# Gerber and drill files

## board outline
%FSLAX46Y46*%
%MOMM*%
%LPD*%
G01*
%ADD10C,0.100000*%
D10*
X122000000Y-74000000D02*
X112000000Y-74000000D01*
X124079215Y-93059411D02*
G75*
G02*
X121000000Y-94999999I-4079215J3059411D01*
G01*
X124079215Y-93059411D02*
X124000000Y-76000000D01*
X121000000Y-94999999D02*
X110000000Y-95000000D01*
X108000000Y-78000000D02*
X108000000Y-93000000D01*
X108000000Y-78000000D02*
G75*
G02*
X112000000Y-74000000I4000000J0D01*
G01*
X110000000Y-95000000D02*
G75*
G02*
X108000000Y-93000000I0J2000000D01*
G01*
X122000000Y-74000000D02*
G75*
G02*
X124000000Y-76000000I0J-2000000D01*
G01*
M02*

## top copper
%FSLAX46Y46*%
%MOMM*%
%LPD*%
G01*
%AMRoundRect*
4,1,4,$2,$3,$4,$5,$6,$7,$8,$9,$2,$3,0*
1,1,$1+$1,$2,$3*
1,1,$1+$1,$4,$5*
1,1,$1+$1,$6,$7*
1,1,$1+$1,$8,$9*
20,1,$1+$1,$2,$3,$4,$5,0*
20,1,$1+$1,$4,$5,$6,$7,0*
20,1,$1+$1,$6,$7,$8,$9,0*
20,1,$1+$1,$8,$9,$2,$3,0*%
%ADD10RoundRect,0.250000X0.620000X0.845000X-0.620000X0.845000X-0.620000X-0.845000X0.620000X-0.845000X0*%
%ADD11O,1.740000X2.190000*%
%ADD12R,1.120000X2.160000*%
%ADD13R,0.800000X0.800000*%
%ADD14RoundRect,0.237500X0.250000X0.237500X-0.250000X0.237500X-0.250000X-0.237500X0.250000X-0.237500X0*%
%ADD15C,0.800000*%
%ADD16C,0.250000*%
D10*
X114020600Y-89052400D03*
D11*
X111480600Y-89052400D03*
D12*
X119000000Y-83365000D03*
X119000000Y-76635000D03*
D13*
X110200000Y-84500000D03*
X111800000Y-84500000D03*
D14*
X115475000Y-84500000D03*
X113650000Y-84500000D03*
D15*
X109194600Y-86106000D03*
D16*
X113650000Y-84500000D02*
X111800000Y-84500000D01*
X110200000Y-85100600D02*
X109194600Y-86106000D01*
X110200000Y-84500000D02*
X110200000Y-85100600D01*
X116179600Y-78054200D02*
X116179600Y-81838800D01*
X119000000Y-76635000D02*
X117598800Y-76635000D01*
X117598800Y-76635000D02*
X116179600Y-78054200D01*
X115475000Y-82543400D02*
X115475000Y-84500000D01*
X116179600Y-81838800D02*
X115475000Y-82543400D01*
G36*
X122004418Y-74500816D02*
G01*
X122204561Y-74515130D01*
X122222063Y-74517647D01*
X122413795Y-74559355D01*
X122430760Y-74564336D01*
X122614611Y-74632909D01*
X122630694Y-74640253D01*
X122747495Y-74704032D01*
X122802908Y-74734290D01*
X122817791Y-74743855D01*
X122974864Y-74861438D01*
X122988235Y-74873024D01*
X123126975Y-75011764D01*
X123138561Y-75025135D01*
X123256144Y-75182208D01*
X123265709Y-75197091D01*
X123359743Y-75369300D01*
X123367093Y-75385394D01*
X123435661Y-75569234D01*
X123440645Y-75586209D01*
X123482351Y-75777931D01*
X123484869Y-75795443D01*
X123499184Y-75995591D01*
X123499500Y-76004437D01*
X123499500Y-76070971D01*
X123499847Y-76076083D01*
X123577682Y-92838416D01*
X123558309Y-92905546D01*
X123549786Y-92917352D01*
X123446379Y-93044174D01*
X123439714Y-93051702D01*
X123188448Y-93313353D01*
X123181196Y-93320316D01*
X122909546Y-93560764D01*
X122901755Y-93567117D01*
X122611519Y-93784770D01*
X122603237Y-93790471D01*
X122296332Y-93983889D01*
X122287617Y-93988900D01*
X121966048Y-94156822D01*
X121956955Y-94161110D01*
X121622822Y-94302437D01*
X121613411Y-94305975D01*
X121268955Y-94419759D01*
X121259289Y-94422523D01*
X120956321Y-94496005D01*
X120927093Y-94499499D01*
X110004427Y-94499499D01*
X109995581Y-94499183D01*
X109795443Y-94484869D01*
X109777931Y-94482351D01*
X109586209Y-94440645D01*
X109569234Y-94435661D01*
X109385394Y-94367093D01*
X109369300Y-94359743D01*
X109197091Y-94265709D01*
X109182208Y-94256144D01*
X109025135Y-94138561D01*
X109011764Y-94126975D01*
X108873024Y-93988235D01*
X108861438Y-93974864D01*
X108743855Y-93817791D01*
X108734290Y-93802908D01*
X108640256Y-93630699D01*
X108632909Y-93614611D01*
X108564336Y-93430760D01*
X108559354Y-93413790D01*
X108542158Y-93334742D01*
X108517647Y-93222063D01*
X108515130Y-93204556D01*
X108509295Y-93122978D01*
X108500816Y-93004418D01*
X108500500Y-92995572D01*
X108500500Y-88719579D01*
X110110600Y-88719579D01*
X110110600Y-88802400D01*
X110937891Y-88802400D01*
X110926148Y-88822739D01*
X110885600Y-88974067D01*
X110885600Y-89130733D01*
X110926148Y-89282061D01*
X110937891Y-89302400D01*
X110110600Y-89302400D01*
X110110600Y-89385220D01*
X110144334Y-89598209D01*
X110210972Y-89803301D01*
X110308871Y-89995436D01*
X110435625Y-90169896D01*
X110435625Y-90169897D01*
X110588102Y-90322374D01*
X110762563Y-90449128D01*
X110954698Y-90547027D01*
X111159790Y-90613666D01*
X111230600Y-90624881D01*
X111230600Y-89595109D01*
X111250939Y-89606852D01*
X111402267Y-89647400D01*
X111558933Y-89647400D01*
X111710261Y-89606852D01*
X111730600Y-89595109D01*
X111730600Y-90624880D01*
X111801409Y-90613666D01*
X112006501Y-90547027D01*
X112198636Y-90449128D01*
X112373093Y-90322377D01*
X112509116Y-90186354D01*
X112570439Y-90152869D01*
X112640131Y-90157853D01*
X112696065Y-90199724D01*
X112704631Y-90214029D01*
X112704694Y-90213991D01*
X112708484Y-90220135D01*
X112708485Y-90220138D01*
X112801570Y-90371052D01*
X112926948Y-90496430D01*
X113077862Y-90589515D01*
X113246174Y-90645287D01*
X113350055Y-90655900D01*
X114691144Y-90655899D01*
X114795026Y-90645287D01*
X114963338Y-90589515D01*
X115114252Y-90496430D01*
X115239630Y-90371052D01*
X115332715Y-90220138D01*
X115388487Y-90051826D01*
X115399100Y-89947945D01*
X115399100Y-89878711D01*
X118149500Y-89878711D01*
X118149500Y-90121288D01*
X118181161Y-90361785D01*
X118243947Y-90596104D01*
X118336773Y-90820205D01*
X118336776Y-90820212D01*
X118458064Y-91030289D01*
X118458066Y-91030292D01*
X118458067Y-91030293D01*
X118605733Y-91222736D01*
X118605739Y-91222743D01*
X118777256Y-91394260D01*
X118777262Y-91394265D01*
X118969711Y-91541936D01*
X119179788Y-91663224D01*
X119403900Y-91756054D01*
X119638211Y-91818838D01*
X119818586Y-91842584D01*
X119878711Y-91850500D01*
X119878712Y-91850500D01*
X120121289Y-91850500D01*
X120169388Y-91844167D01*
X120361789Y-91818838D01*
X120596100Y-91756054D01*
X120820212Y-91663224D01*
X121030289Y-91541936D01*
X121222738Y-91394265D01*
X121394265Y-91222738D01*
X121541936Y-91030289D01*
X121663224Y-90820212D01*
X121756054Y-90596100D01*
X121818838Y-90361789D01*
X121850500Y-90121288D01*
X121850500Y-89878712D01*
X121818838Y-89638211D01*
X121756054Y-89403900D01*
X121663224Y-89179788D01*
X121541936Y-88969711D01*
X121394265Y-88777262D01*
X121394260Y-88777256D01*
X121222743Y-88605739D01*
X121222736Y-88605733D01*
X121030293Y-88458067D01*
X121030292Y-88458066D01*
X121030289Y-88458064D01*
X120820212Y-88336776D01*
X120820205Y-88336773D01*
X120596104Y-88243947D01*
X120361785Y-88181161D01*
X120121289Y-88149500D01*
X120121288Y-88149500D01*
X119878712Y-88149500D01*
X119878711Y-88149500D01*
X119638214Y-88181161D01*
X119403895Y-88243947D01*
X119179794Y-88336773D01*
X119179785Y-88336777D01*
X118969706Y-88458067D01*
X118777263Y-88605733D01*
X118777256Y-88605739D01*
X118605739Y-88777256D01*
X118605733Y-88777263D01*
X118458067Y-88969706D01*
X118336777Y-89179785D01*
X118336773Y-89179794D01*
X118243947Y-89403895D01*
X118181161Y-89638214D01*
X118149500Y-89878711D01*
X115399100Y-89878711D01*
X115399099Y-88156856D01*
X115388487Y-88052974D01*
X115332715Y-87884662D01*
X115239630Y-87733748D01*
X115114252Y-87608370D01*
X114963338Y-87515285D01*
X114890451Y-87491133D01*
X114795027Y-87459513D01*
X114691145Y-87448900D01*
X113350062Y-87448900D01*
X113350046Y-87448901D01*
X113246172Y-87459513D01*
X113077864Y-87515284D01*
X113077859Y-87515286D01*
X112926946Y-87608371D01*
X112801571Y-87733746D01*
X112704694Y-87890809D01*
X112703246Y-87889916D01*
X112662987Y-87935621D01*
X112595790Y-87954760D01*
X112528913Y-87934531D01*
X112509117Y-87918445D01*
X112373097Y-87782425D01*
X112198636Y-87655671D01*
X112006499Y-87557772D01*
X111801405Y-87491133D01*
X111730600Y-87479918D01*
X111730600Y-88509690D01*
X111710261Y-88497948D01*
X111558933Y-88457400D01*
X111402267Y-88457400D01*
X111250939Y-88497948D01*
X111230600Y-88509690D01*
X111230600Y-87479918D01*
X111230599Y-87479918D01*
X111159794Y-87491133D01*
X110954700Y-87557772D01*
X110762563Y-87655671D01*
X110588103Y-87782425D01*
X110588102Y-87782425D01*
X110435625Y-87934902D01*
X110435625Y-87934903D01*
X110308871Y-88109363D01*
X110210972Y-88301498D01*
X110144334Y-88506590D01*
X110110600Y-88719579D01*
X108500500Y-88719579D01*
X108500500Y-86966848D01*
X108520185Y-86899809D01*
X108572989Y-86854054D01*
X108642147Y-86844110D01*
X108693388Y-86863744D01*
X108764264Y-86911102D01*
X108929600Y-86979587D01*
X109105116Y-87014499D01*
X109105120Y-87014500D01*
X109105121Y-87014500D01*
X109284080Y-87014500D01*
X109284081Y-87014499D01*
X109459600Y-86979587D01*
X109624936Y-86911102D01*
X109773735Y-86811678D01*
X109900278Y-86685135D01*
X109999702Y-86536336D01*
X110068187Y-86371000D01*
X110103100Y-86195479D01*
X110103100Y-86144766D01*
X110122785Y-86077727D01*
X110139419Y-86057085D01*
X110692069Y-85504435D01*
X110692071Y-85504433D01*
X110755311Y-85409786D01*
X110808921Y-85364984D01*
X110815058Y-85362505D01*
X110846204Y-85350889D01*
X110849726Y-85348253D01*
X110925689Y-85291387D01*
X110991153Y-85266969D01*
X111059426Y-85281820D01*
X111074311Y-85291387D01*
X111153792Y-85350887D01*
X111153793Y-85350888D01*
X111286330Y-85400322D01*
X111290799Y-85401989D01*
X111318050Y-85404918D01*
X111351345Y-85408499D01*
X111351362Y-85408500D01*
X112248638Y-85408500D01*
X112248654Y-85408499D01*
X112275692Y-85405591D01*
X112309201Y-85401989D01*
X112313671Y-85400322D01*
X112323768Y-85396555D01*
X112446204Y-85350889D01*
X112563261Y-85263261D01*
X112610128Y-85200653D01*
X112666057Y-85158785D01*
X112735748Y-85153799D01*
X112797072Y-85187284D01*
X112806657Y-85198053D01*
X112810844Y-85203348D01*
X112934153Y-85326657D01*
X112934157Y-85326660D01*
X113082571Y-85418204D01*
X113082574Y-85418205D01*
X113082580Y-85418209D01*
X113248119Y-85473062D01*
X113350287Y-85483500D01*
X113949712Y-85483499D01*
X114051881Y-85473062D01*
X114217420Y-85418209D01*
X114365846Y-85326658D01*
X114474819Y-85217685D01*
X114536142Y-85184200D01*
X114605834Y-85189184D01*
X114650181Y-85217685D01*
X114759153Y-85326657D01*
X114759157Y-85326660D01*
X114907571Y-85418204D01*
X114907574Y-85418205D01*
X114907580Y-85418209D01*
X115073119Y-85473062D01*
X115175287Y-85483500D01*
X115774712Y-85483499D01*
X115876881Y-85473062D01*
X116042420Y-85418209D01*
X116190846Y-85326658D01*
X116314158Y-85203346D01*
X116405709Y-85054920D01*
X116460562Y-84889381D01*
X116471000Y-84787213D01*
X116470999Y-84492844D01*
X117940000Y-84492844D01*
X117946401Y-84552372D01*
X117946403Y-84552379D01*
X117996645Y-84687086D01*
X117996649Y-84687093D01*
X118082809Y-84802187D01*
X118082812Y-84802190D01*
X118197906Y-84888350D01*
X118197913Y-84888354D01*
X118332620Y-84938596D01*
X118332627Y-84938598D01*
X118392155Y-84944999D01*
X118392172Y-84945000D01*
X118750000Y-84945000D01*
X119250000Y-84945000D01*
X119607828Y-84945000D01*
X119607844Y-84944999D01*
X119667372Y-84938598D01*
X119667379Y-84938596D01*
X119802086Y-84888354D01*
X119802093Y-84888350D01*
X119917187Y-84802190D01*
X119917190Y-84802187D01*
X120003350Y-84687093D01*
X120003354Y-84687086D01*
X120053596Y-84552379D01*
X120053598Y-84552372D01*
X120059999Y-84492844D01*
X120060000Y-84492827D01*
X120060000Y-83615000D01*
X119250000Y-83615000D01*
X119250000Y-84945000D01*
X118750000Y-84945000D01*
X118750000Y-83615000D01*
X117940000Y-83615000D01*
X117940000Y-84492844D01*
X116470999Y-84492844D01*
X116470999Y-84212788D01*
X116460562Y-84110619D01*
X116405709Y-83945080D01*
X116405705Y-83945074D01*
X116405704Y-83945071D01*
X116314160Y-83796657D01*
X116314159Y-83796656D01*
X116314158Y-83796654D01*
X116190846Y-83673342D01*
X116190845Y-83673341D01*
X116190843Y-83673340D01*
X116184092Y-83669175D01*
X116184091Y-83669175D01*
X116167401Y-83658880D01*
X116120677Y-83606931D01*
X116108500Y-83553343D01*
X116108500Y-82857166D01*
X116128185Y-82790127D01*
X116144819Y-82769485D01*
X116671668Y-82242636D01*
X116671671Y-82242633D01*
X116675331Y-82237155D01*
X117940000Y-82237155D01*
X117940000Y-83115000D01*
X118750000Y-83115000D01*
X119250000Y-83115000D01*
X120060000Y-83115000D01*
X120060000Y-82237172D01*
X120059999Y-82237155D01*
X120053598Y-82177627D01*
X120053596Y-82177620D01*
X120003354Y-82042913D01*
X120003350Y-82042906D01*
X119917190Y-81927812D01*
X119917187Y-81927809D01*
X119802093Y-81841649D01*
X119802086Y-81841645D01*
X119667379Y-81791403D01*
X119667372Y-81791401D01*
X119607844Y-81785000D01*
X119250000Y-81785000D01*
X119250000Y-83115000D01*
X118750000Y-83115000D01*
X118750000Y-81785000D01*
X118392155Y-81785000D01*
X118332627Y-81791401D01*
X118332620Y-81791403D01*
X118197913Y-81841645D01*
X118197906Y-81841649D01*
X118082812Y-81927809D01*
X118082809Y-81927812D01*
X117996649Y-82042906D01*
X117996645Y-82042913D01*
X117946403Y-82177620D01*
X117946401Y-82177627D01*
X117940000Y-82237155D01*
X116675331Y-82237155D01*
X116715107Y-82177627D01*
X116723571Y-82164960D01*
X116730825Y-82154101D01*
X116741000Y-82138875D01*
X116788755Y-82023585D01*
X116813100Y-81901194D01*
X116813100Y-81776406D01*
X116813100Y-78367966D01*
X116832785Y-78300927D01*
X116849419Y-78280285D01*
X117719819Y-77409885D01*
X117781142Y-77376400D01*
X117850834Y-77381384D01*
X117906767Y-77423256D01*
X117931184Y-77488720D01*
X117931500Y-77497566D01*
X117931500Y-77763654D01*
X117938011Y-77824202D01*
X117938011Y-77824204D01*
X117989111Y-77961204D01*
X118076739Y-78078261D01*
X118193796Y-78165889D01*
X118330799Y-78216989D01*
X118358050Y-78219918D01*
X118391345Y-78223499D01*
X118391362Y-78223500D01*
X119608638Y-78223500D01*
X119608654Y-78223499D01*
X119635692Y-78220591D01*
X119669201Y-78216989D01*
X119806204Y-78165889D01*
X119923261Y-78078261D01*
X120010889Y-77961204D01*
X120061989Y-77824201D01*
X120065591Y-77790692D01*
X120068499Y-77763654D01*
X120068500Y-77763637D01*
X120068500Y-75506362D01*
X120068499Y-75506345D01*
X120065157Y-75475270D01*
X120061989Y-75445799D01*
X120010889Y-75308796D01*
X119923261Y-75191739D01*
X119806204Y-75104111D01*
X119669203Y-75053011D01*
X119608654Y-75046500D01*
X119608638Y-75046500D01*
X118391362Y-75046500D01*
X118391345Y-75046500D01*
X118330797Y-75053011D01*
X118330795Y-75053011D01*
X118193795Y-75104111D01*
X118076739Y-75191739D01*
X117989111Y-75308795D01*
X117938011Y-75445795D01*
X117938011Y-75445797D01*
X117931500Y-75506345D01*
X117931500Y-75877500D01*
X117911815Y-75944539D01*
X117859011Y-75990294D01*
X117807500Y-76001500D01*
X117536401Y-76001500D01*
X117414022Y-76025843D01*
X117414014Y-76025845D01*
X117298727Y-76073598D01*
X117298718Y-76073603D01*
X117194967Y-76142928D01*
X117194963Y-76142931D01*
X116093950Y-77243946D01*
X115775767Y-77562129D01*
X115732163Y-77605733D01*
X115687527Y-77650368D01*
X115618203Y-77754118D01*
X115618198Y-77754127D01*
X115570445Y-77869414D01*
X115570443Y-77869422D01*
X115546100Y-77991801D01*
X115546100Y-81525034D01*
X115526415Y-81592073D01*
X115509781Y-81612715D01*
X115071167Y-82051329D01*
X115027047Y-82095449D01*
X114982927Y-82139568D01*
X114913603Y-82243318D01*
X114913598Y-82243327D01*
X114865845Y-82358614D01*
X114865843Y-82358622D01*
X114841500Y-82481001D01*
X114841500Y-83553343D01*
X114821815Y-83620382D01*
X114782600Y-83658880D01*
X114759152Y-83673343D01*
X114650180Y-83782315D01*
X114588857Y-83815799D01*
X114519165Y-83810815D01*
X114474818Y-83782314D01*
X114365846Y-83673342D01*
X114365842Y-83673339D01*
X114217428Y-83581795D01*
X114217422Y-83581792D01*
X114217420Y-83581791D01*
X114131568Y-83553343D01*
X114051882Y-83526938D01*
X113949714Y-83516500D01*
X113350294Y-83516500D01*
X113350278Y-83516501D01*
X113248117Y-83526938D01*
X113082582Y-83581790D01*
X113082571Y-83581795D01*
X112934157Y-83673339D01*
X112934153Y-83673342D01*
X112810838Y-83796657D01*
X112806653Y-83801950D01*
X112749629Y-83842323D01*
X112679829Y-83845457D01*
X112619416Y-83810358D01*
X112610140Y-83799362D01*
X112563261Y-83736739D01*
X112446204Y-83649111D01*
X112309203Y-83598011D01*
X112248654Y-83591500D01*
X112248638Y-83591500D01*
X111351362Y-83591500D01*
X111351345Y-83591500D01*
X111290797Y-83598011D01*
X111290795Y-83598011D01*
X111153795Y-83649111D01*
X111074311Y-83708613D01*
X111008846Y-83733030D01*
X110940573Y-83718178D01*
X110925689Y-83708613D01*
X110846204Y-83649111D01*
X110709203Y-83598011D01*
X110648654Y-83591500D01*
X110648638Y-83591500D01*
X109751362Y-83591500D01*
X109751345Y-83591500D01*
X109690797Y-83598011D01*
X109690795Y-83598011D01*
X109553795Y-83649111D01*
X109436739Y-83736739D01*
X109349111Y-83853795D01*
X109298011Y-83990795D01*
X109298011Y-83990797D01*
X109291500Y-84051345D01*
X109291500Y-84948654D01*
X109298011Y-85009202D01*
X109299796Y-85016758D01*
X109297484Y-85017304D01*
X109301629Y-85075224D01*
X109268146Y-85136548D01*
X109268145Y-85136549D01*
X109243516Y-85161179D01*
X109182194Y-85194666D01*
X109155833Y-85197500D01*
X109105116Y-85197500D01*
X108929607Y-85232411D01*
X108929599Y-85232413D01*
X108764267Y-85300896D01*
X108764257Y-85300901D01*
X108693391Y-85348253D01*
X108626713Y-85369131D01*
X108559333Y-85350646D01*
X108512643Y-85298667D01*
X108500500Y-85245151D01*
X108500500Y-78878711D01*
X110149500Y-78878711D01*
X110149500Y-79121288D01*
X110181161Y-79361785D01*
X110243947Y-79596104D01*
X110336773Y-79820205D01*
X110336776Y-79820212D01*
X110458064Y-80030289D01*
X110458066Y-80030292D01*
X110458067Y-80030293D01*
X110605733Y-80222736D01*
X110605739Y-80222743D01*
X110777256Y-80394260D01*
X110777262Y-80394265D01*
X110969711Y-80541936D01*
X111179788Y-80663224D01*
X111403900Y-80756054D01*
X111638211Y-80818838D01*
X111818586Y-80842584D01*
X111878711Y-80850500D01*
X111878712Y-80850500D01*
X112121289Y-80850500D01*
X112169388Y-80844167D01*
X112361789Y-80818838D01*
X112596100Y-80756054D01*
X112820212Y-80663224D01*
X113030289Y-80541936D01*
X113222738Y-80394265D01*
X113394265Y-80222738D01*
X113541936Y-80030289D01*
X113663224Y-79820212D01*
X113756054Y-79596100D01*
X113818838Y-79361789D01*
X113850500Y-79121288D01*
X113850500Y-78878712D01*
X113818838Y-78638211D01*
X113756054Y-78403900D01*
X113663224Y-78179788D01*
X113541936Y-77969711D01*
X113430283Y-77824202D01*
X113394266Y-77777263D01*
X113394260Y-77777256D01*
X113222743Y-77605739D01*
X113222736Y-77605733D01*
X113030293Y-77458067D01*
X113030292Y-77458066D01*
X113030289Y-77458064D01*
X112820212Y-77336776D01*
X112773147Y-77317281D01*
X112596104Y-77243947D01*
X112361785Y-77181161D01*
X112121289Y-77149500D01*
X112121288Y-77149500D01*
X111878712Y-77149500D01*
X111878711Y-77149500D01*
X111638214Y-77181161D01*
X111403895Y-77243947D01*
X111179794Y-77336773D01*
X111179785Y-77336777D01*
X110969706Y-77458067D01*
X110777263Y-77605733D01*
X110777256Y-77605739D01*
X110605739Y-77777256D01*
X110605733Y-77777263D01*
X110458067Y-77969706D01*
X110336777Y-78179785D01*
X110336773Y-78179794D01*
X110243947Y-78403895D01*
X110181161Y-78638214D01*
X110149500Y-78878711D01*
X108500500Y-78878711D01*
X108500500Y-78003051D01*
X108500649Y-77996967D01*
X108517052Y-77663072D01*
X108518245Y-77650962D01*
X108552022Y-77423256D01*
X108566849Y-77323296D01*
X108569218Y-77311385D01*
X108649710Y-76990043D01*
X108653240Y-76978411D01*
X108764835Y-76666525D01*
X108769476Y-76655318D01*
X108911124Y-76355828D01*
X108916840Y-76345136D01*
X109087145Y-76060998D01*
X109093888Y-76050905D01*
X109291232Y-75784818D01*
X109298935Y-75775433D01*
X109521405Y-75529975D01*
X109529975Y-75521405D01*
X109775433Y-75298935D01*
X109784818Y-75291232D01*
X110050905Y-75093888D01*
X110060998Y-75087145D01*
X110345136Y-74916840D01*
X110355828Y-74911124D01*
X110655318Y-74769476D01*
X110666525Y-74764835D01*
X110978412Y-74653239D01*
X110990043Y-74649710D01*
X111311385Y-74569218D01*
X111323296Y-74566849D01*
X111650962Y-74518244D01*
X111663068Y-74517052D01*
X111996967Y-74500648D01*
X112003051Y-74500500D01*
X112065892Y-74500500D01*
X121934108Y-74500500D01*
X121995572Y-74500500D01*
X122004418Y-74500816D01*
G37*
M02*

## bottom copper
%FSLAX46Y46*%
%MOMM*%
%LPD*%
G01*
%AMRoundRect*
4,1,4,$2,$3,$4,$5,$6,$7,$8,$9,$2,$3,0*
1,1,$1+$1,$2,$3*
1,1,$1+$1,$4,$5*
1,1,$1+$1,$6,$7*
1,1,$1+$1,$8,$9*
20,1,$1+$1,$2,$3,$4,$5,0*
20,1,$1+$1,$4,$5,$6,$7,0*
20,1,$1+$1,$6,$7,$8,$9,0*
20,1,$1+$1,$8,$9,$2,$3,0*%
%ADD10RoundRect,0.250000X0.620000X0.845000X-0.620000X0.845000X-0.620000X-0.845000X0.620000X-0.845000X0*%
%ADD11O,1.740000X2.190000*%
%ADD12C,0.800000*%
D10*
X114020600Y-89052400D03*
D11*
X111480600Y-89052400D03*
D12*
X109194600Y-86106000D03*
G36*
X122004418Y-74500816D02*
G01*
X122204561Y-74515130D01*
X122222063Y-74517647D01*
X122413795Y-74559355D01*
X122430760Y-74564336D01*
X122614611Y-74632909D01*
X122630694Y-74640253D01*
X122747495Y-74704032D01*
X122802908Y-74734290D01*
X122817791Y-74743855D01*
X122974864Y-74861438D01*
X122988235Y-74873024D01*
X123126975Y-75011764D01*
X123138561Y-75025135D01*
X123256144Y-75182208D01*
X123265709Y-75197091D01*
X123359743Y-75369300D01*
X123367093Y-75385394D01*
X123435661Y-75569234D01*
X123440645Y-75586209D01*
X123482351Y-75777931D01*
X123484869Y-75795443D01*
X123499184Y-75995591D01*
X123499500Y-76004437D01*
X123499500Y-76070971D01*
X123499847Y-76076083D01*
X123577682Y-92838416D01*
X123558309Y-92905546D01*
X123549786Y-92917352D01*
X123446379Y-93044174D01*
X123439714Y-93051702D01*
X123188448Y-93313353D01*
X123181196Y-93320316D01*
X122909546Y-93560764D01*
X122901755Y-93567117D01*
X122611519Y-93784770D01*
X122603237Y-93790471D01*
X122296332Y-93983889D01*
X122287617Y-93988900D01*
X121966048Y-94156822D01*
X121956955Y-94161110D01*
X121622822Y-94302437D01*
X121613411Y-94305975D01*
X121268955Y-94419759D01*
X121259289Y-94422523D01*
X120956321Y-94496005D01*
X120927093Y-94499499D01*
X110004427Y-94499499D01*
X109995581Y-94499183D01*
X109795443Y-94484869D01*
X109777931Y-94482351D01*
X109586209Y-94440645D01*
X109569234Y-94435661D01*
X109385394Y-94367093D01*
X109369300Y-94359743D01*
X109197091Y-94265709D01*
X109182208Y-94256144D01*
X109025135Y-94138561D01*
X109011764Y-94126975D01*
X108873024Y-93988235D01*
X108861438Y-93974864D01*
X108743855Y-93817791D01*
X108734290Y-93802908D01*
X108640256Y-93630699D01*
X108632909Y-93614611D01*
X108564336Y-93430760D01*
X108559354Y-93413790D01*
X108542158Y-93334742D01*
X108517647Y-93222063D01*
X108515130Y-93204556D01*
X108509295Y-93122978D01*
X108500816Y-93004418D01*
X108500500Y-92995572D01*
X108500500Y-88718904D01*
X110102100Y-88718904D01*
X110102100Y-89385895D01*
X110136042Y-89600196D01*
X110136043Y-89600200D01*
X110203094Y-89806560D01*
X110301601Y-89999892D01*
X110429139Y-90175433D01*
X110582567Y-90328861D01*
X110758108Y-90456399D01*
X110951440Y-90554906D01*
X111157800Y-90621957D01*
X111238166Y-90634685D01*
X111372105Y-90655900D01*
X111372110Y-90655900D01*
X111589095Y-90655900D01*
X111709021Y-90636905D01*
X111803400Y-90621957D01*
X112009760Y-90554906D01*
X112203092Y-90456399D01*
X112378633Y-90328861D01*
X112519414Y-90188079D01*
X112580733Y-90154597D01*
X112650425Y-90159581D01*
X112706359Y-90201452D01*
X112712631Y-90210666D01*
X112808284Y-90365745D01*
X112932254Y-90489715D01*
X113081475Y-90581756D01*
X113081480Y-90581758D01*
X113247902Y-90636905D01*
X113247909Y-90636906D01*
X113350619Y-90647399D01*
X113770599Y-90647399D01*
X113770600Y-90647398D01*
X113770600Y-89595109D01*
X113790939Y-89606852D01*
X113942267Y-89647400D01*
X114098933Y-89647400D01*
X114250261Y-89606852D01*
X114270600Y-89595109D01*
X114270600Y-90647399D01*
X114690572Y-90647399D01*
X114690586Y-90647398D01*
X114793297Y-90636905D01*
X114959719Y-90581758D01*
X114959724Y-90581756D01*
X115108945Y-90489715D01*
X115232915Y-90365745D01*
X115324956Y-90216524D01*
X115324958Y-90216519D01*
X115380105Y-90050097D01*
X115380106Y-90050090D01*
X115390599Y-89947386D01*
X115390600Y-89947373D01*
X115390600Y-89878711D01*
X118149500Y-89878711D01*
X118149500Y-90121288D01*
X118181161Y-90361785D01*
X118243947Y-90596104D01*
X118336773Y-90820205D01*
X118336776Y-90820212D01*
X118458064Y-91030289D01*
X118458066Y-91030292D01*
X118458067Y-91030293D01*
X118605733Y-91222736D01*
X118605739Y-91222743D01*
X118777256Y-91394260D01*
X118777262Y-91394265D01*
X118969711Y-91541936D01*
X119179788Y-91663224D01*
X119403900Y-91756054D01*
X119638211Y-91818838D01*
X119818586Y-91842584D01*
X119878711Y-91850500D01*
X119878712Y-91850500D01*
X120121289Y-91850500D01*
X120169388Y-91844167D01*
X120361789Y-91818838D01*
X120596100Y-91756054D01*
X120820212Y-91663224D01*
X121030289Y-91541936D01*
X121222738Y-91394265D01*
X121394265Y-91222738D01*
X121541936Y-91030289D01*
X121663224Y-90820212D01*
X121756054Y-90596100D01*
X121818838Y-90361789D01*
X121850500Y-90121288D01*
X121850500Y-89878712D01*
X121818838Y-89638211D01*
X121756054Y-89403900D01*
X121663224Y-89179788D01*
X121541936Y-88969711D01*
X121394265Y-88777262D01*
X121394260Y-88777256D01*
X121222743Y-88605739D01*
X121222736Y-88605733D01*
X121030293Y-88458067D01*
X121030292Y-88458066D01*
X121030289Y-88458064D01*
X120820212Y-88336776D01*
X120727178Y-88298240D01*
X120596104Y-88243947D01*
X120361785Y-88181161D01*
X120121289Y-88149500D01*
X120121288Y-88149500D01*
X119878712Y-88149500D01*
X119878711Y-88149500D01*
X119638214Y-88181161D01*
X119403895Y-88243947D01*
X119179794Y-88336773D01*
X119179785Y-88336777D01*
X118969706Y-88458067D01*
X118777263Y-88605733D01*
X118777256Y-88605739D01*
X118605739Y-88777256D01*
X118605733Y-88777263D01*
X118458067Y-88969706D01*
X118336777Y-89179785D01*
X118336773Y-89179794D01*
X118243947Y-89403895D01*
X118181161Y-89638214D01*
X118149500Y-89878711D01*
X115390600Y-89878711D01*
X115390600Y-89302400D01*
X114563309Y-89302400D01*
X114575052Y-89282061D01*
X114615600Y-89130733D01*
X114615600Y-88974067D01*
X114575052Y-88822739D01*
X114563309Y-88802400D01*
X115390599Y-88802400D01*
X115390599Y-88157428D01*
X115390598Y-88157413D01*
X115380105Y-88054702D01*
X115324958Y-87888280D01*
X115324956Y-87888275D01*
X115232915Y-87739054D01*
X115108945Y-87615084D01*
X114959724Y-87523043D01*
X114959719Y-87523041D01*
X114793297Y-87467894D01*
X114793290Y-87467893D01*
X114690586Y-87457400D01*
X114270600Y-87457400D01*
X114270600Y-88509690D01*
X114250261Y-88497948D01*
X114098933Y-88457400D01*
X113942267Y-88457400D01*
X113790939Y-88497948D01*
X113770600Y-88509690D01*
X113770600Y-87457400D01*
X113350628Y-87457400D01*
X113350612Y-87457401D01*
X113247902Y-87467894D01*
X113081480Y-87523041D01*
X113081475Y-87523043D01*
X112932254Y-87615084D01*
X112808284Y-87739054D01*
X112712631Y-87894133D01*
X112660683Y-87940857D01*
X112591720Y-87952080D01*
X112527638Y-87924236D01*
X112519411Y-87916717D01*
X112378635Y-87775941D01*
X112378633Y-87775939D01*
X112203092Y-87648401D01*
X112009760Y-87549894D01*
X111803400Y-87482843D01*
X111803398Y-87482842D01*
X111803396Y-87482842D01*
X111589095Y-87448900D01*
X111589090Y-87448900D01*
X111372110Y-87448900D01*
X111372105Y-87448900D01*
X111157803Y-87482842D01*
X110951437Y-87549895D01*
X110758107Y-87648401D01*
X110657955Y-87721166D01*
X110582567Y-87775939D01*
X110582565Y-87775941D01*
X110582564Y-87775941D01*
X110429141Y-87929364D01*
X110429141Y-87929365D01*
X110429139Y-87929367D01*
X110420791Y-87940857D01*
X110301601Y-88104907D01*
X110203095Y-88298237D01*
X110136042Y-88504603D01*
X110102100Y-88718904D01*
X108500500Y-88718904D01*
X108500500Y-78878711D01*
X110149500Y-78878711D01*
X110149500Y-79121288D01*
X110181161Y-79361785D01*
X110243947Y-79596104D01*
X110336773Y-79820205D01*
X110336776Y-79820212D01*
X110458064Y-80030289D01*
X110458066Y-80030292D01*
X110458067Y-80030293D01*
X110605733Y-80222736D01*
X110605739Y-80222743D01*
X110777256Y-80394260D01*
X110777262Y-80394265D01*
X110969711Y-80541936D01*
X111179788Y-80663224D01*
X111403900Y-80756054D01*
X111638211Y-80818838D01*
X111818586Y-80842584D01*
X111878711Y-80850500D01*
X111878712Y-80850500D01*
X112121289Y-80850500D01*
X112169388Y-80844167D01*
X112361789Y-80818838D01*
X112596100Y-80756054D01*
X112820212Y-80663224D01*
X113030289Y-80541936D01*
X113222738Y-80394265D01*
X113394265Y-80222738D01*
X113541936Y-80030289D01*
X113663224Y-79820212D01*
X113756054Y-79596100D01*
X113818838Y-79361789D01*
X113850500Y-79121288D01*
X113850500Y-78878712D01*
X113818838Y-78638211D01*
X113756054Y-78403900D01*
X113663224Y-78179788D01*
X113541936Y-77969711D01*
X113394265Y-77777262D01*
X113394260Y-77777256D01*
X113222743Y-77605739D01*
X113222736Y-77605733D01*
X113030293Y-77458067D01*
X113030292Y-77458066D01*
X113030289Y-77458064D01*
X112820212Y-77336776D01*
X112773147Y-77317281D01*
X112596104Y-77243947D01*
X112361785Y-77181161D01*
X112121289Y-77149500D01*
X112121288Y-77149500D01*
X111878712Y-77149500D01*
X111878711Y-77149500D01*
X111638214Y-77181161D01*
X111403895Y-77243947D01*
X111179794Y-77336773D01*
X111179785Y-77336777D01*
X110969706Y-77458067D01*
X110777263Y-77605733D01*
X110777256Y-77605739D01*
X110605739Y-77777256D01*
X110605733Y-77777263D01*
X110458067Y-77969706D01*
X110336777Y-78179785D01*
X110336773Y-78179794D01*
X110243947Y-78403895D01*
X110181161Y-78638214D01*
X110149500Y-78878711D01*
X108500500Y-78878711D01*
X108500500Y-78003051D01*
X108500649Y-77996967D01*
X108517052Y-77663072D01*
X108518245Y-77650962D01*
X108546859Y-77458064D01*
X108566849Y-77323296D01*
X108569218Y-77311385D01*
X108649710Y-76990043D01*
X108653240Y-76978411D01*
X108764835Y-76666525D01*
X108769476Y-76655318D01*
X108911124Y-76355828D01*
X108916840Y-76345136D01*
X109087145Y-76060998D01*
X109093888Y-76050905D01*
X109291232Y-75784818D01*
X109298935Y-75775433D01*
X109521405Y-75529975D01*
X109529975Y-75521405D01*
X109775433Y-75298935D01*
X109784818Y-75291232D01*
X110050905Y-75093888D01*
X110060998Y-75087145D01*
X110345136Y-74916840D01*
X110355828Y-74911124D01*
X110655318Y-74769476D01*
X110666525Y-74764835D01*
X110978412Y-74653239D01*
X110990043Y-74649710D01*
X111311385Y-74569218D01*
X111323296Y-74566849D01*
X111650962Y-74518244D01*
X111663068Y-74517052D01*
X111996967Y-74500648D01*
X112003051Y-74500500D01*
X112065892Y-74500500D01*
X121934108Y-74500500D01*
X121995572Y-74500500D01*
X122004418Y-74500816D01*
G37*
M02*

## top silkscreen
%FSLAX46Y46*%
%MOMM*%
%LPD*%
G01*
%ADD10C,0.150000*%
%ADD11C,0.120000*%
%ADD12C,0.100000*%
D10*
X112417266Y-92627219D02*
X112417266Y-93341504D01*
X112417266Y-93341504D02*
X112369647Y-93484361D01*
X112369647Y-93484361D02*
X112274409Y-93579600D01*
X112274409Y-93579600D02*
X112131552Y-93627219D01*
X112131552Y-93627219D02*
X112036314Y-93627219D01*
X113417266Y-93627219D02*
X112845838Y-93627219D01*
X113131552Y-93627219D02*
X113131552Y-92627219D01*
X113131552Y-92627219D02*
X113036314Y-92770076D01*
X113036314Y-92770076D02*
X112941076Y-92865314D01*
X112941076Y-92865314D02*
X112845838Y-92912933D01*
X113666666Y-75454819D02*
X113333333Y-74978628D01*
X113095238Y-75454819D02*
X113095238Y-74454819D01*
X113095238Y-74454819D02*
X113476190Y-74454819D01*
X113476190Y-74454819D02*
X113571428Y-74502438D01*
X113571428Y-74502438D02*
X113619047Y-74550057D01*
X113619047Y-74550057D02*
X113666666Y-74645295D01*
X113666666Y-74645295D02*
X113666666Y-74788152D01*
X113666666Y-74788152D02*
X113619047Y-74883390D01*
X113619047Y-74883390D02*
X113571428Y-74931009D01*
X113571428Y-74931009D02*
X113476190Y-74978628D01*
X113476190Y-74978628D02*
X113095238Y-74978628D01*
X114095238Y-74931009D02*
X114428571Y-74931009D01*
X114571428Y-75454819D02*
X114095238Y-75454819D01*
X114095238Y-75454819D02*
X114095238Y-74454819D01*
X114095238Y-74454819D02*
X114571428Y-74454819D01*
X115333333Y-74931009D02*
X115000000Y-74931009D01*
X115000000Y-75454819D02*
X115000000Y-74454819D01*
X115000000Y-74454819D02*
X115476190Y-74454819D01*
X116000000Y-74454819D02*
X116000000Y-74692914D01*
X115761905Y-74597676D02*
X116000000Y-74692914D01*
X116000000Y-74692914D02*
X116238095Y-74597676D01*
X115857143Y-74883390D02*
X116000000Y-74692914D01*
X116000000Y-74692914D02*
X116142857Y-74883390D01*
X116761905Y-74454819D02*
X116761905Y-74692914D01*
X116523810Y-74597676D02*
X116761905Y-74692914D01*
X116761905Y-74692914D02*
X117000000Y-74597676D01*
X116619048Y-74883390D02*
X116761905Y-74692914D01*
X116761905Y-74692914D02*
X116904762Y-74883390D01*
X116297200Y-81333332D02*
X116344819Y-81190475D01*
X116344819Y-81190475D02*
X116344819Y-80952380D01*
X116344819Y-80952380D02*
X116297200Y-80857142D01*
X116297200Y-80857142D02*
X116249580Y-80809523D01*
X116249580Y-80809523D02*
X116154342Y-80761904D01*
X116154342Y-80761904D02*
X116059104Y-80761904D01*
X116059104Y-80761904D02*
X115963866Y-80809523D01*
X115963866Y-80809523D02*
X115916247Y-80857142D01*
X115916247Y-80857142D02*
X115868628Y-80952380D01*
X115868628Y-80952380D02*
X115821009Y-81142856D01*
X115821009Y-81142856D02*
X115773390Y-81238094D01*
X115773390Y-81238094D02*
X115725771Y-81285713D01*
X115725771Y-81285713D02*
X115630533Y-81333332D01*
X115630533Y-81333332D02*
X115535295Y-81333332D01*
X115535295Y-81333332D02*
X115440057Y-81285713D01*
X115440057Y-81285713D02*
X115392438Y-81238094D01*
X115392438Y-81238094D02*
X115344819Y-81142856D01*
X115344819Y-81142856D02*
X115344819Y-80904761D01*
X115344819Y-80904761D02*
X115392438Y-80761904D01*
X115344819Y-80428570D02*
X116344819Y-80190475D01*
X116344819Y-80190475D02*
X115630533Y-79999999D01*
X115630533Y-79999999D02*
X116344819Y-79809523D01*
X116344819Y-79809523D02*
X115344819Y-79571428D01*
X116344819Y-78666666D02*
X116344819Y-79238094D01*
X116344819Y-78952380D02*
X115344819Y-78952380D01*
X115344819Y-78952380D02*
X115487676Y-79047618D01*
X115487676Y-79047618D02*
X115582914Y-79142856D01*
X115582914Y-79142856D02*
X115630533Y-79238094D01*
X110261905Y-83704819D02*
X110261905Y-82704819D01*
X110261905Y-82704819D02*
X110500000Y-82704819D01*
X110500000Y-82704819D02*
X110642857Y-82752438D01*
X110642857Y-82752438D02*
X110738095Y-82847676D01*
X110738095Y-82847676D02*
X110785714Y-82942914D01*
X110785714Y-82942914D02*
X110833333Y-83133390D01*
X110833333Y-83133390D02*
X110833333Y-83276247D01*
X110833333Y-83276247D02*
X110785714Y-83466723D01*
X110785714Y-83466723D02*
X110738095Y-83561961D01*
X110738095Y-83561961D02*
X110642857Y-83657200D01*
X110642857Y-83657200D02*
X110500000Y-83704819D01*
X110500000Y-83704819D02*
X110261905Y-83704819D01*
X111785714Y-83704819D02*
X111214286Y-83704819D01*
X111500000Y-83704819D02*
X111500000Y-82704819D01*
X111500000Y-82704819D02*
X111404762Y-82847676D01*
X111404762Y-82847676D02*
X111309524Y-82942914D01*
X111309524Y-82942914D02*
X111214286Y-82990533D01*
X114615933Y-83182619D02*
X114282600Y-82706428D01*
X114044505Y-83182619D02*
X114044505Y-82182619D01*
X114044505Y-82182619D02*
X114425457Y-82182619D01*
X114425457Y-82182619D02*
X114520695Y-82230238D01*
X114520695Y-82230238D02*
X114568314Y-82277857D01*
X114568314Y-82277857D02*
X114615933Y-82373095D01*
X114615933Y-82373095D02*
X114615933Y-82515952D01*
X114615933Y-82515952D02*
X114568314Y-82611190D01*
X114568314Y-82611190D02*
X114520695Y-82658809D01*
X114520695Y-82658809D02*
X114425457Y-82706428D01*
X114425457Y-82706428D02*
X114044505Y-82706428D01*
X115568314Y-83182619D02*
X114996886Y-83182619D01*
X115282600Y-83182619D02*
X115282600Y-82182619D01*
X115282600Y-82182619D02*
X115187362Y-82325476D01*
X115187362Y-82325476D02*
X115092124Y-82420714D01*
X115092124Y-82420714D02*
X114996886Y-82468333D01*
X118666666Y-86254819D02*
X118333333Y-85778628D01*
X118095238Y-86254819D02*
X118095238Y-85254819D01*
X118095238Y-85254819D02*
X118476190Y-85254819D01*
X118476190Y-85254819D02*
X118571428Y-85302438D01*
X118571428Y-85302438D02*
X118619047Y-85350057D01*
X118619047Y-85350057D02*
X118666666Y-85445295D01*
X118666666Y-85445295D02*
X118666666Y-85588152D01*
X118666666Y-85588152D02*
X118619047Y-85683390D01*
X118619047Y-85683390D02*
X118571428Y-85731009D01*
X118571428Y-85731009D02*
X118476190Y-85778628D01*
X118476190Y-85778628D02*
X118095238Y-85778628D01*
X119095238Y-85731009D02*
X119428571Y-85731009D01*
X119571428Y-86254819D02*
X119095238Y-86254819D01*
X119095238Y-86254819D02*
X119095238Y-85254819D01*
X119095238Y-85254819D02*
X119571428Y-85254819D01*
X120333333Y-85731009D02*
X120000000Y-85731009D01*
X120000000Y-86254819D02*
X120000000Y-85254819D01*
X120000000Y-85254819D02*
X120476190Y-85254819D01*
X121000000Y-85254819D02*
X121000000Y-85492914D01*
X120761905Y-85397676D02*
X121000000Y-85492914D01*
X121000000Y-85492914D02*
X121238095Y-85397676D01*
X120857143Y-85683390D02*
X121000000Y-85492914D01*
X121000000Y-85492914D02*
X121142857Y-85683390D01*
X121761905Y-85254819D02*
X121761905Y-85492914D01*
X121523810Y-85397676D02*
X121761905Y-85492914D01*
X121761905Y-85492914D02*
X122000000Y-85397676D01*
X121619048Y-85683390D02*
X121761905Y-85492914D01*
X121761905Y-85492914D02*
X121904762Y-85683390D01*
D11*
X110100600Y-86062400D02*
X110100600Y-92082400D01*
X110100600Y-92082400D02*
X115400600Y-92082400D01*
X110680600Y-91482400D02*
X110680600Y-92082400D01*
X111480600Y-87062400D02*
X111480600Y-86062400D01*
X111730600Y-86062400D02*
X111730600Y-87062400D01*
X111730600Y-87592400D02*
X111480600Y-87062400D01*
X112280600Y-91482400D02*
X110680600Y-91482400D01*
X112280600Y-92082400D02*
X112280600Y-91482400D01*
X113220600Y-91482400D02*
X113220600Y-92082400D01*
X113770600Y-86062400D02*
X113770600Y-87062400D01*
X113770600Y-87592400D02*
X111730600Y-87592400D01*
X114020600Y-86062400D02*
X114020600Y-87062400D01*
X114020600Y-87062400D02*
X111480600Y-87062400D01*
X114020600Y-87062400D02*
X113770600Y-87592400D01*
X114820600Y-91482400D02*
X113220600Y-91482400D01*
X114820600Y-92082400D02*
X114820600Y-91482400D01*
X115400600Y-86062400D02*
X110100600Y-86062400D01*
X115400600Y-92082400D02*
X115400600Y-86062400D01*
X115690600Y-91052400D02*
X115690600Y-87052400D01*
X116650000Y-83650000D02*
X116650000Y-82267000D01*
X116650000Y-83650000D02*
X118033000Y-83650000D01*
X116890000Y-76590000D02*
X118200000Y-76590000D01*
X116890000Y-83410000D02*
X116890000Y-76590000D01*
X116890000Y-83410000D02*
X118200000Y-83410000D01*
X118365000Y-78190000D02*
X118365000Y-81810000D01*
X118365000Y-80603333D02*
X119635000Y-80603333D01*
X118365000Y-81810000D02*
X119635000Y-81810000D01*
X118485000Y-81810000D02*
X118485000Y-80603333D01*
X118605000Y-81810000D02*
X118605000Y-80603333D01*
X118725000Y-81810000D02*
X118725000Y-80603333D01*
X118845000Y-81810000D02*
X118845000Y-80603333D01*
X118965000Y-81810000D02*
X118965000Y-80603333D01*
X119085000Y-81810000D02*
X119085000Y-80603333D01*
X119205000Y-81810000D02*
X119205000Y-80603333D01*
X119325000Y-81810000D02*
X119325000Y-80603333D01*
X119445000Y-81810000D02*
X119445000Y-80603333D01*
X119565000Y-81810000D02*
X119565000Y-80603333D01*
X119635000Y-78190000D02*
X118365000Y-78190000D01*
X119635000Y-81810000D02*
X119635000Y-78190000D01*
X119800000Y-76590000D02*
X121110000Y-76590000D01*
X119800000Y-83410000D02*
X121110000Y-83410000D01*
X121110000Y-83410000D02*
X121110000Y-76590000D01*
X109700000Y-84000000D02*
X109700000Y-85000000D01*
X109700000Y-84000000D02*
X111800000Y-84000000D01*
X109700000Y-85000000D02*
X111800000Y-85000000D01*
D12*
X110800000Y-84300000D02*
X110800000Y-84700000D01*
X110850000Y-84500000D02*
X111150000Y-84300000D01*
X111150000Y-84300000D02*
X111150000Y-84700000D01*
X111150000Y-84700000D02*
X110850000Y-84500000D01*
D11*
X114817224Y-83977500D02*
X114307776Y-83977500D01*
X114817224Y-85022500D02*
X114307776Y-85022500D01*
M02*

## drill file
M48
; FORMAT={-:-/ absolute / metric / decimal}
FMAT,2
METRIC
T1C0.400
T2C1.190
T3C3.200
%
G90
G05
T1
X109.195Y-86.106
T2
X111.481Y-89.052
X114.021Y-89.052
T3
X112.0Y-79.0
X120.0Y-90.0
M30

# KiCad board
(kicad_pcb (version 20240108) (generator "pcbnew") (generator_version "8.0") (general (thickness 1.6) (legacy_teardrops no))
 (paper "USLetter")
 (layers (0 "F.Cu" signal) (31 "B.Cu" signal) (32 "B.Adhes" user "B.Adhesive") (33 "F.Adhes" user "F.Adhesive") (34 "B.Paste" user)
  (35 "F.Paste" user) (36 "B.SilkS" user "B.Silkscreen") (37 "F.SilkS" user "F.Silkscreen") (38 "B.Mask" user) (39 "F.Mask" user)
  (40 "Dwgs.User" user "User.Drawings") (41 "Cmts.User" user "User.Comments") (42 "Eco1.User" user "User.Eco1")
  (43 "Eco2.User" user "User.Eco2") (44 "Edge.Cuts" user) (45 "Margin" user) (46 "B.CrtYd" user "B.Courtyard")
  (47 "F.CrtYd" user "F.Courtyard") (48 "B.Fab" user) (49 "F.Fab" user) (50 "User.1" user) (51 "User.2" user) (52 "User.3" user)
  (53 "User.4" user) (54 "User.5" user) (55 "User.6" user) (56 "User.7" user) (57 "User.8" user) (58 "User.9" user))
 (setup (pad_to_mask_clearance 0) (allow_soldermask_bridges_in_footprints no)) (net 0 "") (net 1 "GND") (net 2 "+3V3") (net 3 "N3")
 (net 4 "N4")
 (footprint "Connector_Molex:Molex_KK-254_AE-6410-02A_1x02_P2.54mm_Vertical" (layer "F.Cu") (at 114.0206 89.0524 180)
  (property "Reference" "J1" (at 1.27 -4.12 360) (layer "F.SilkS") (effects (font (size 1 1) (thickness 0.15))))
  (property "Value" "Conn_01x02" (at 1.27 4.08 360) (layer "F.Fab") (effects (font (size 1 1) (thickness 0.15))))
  (fp_line (start 3.92 2.99) (end 3.92 -3.03) (stroke (width 0.12) (type solid)) (layer "F.SilkS"))
  (fp_line (start 3.92 -3.03) (end -1.38 -3.03) (stroke (width 0.12) (type solid)) (layer "F.SilkS"))
  (fp_line (start 3.34 -2.43) (end 3.34 -3.03) (stroke (width 0.12) (type solid)) (layer "F.SilkS"))
  (fp_line (start 2.54 1.99) (end 2.54 2.99) (stroke (width 0.12) (type solid)) (layer "F.SilkS"))
  (fp_line (start 2.29 2.99) (end 2.29 1.99) (stroke (width 0.12) (type solid)) (layer "F.SilkS"))
  (fp_line (start 2.29 1.46) (end 2.54 1.99) (stroke (width 0.12) (type solid)) (layer "F.SilkS"))
  (fp_line (start 1.74 -2.43) (end 3.34 -2.43) (stroke (width 0.12) (type solid)) (layer "F.SilkS"))
  (fp_line (start 1.74 -3.03) (end 1.74 -2.43) (stroke (width 0.12) (type solid)) (layer "F.SilkS"))
  (fp_line (start 0.8 -2.43) (end 0.8 -3.03) (stroke (width 0.12) (type solid)) (layer "F.SilkS"))
  (fp_line (start 0.25 2.99) (end 0.25 1.99) (stroke (width 0.12) (type solid)) (layer "F.SilkS"))
  (fp_line (start 0.25 1.46) (end 2.29 1.46) (stroke (width 0.12) (type solid)) (layer "F.SilkS"))
  (fp_line (start 0 2.99) (end 0 1.99) (stroke (width 0.12) (type solid)) (layer "F.SilkS"))
  (fp_line (start 0 1.99) (end 2.54 1.99) (stroke (width 0.12) (type solid)) (layer "F.SilkS"))
  (fp_line (start 0 1.99) (end 0.25 1.46) (stroke (width 0.12) (type solid)) (layer "F.SilkS"))
  (fp_line (start -0.8 -2.43) (end 0.8 -2.43) (stroke (width 0.12) (type solid)) (layer "F.SilkS"))
  (fp_line (start -0.8 -3.03) (end -0.8 -2.43) (stroke (width 0.12) (type solid)) (layer "F.SilkS"))
  (fp_line (start -1.38 2.99) (end 3.92 2.99) (stroke (width 0.12) (type solid)) (layer "F.SilkS"))
  (fp_line (start -1.38 -3.03) (end -1.38 2.99) (stroke (width 0.12) (type solid)) (layer "F.SilkS"))
  (fp_line (start -1.67 -2) (end -1.67 2) (stroke (width 0.12) (type solid)) (layer "F.SilkS"))
  (pad "1" thru_hole roundrect (at 0 0 180) (size 1.74 2.19) (drill 1.19) (layers "*.Cu" "*.Mask") (remove_unused_layers no)
   (roundrect_rratio 0.143678) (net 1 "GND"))
  (pad "2" thru_hole oval (at 2.54 0 180) (size 1.74 2.19) (drill 1.19) (layers "*.Cu" "*.Mask") (remove_unused_layers no) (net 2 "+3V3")))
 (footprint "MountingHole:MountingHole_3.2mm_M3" (layer "F.Cu") (at 112 79)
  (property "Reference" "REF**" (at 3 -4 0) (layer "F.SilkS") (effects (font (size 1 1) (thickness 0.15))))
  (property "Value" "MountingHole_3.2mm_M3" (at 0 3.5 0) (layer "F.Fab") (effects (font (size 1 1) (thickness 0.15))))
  (pad "" np_thru_hole circle (at 0 0) (size 3.2 3.2) (drill 3.2) (layers "*.Cu" "*.Mask")))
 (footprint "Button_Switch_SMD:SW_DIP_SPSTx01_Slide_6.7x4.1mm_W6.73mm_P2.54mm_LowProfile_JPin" (layer "F.Cu") (at 119 80 90)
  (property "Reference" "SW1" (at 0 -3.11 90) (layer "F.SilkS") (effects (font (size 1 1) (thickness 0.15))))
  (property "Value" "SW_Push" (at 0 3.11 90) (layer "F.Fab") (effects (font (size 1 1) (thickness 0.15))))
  (fp_line (start -3.65 -2.35) (end -2.267 -2.35) (stroke (width 0.12) (type solid)) (layer "F.SilkS"))
  (fp_line (start -3.65 -2.35) (end -3.65 -0.967) (stroke (width 0.12) (type solid)) (layer "F.SilkS"))
  (fp_line (start 3.41 -2.11) (end 3.41 -0.8) (stroke (width 0.12) (type solid)) (layer "F.SilkS"))
  (fp_line (start -3.41 -2.11) (end 3.41 -2.11) (stroke (width 0.12) (type solid)) (layer "F.SilkS"))
  (fp_line (start -3.41 -2.11) (end -3.41 -0.8) (stroke (width 0.12) (type solid)) (layer "F.SilkS"))
  (fp_line (start 1.81 -0.635) (end -1.81 -0.635) (stroke (width 0.12) (type solid)) (layer "F.SilkS"))
  (fp_line (start -0.603333 -0.635) (end -0.603333 0.635) (stroke (width 0.12) (type solid)) (layer "F.SilkS"))
  (fp_line (start -1.81 -0.635) (end -1.81 0.635) (stroke (width 0.12) (type solid)) (layer "F.SilkS"))
  (fp_line (start -1.81 -0.515) (end -0.603333 -0.515) (stroke (width 0.12) (type solid)) (layer "F.SilkS"))
  (fp_line (start -1.81 -0.395) (end -0.603333 -0.395) (stroke (width 0.12) (type solid)) (layer "F.SilkS"))
  (fp_line (start -1.81 -0.275) (end -0.603333 -0.275) (stroke (width 0.12) (type solid)) (layer "F.SilkS"))
  (fp_line (start -1.81 -0.155) (end -0.603333 -0.155) (stroke (width 0.12) (type solid)) (layer "F.SilkS"))
  (fp_line (start -1.81 -0.035) (end -0.603333 -0.035) (stroke (width 0.12) (type solid)) (layer "F.SilkS"))
  (fp_line (start -1.81 0.085) (end -0.603333 0.085) (stroke (width 0.12) (type solid)) (layer "F.SilkS"))
  (fp_line (start -1.81 0.205) (end -0.603333 0.205) (stroke (width 0.12) (type solid)) (layer "F.SilkS"))
  (fp_line (start -1.81 0.325) (end -0.603333 0.325) (stroke (width 0.12) (type solid)) (layer "F.SilkS"))
  (fp_line (start -1.81 0.445) (end -0.603333 0.445) (stroke (width 0.12) (type solid)) (layer "F.SilkS"))
  (fp_line (start -1.81 0.565) (end -0.603333 0.565) (stroke (width 0.12) (type solid)) (layer "F.SilkS"))
  (fp_line (start 1.81 0.635) (end 1.81 -0.635) (stroke (width 0.12) (type solid)) (layer "F.SilkS"))
  (fp_line (start -1.81 0.635) (end 1.81 0.635) (stroke (width 0.12) (type solid)) (layer "F.SilkS"))
  (fp_line (start 3.41 0.8) (end 3.41 2.11) (stroke (width 0.12) (type solid)) (layer "F.SilkS"))
  (fp_line (start -3.41 0.8) (end -3.41 2.11) (stroke (width 0.12) (type solid)) (layer "F.SilkS"))
  (fp_line (start -3.41 2.11) (end 3.41 2.11) (stroke (width 0.12) (type solid)) (layer "F.SilkS"))
  (pad "1" smd rect (at -3.365 0 90) (size 2.16 1.12) (layers "F.Cu" "F.Paste" "F.Mask") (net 2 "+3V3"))
  (pad "2" smd rect (at 3.365 0 90) (size 2.16 1.12) (layers "F.Cu" "F.Paste" "F.Mask") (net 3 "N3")))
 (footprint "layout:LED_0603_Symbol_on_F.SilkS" (layer "F.Cu") (at 111 84.5)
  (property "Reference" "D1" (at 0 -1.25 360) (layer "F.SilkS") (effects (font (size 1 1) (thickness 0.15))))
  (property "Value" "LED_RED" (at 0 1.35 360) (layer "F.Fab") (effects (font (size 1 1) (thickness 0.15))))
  (fp_line (start -1.3 -0.5) (end -1.3 0.5) (stroke (width 0.12) (type solid)) (layer "F.SilkS"))
  (fp_line (start -1.3 -0.5) (end 0.8 -0.5) (stroke (width 0.12) (type solid)) (layer "F.SilkS"))
  (fp_line (start -1.3 0.5) (end 0.8 0.5) (stroke (width 0.12) (type solid)) (layer "F.SilkS"))
  (fp_line (start -0.2 -0.2) (end -0.2 0.2) (stroke (width 0.1) (type solid)) (layer "F.SilkS"))
  (fp_line (start -0.15 0) (end 0.15 -0.2) (stroke (width 0.1) (type solid)) (layer "F.SilkS"))
  (fp_line (start 0.15 -0.2) (end 0.15 0.2) (stroke (width 0.1) (type solid)) (layer "F.SilkS"))
  (fp_line (start 0.15 0.2) (end -0.15 0) (stroke (width 0.1) (type solid)) (layer "F.SilkS"))
  (pad "1" smd rect (at -0.8 0 180) (size 0.8 0.8) (layers "F.Cu" "F.Paste" "F.Mask") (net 1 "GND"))
  (pad "2" smd rect (at 0.8 0 180) (size 0.8 0.8) (layers "F.Cu" "F.Paste" "F.Mask") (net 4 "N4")))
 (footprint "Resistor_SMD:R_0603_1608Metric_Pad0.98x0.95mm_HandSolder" (layer "F.Cu") (at 114.5625 84.5 180)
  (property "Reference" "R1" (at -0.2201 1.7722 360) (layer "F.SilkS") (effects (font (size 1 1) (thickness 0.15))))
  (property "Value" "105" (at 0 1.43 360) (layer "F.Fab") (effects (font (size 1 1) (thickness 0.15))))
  (fp_line (start -0.254724 0.5225) (end 0.254724 0.5225) (stroke (width 0.12) (type solid)) (layer "F.SilkS"))
  (fp_line (start -0.254724 -0.5225) (end 0.254724 -0.5225) (stroke (width 0.12) (type solid)) (layer "F.SilkS"))
  (pad "1" smd roundrect (at -0.9125 0 180) (size 0.975 0.95) (layers "F.Cu" "F.Paste" "F.Mask") (roundrect_rratio 0.25) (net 3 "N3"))
  (pad "2" smd roundrect (at 0.9125 0 180) (size 0.975 0.95) (layers "F.Cu" "F.Paste" "F.Mask") (roundrect_rratio 0.25) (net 4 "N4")))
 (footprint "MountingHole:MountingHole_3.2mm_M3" (layer "F.Cu") (at 120 90)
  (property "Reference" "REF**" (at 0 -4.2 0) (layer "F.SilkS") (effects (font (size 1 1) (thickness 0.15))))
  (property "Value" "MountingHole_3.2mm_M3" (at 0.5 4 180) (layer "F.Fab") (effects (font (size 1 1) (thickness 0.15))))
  (pad "" np_thru_hole circle (at 0 0) (size 3.2 3.2) (drill 3.2) (layers "*.Cu" "*.Mask")))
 (gr_line (start 122 74) (end 112 74) (stroke (width 0.1) (type default)) (layer "Edge.Cuts"))
 (gr_arc (start 124.079215 93.059411) (mid 122.718653 94.313805) (end 121 94.999999) (stroke (width 0.1) (type default)) (layer "Edge.Cuts"))
 (gr_line (start 124.079215 93.059411) (end 124 76) (stroke (width 0.1) (type default)) (layer "Edge.Cuts"))
 (gr_line (start 121 94.999999) (end 110 95) (stroke (width 0.1) (type default)) (layer "Edge.Cuts"))
 (gr_line (start 108 78) (end 108 93) (stroke (width 0.1) (type default)) (layer "Edge.Cuts"))
 (gr_arc (start 108 78) (mid 109.171573 75.171573) (end 112 74) (stroke (width 0.1) (type default)) (layer "Edge.Cuts"))
 (gr_arc (start 110 95) (mid 108.585786 94.414214) (end 108 93) (stroke (width 0.1) (type default)) (layer "Edge.Cuts"))
 (gr_arc (start 122 74) (mid 123.414214 74.585786) (end 124 76) (stroke (width 0.1) (type default)) (layer "Edge.Cuts"))
 (segment (start 113.65 84.5) (end 111.8 84.5) (width 0.25) (layer "F.Cu") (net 4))
 (segment (start 110.2 85.1006) (end 109.1946 86.106) (width 0.25) (layer "F.Cu") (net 1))
 (segment (start 110.2 84.5) (end 110.2 85.1006) (width 0.25) (layer "F.Cu") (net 1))
 (via (at 109.1946 86.106) (size 0.8) (drill 0.4) (layers "F.Cu" "B.Cu") (free yes) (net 1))
 (segment (start 116.1796 78.0542) (end 116.1796 81.8388) (width 0.25) (layer "F.Cu") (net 3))
 (segment (start 119 76.635) (end 117.5988 76.635) (width 0.25) (layer "F.Cu") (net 3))
 (segment (start 117.5988 76.635) (end 116.1796 78.0542) (width 0.25) (layer "F.Cu") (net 3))
 (segment (start 115.475 82.5434) (end 115.475 84.5) (width 0.25) (layer "F.Cu") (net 3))
 (segment (start 116.1796 81.8388) (end 115.475 82.5434) (width 0.25) (layer "F.Cu") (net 3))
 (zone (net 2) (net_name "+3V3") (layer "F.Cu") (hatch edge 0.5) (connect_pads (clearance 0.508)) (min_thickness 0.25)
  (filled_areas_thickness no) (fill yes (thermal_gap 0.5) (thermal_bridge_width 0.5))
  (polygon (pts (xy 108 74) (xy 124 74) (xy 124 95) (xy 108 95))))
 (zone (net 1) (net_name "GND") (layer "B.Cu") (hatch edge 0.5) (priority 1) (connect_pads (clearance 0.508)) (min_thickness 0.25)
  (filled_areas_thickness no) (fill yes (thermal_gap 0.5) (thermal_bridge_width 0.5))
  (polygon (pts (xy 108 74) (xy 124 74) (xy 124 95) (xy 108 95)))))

